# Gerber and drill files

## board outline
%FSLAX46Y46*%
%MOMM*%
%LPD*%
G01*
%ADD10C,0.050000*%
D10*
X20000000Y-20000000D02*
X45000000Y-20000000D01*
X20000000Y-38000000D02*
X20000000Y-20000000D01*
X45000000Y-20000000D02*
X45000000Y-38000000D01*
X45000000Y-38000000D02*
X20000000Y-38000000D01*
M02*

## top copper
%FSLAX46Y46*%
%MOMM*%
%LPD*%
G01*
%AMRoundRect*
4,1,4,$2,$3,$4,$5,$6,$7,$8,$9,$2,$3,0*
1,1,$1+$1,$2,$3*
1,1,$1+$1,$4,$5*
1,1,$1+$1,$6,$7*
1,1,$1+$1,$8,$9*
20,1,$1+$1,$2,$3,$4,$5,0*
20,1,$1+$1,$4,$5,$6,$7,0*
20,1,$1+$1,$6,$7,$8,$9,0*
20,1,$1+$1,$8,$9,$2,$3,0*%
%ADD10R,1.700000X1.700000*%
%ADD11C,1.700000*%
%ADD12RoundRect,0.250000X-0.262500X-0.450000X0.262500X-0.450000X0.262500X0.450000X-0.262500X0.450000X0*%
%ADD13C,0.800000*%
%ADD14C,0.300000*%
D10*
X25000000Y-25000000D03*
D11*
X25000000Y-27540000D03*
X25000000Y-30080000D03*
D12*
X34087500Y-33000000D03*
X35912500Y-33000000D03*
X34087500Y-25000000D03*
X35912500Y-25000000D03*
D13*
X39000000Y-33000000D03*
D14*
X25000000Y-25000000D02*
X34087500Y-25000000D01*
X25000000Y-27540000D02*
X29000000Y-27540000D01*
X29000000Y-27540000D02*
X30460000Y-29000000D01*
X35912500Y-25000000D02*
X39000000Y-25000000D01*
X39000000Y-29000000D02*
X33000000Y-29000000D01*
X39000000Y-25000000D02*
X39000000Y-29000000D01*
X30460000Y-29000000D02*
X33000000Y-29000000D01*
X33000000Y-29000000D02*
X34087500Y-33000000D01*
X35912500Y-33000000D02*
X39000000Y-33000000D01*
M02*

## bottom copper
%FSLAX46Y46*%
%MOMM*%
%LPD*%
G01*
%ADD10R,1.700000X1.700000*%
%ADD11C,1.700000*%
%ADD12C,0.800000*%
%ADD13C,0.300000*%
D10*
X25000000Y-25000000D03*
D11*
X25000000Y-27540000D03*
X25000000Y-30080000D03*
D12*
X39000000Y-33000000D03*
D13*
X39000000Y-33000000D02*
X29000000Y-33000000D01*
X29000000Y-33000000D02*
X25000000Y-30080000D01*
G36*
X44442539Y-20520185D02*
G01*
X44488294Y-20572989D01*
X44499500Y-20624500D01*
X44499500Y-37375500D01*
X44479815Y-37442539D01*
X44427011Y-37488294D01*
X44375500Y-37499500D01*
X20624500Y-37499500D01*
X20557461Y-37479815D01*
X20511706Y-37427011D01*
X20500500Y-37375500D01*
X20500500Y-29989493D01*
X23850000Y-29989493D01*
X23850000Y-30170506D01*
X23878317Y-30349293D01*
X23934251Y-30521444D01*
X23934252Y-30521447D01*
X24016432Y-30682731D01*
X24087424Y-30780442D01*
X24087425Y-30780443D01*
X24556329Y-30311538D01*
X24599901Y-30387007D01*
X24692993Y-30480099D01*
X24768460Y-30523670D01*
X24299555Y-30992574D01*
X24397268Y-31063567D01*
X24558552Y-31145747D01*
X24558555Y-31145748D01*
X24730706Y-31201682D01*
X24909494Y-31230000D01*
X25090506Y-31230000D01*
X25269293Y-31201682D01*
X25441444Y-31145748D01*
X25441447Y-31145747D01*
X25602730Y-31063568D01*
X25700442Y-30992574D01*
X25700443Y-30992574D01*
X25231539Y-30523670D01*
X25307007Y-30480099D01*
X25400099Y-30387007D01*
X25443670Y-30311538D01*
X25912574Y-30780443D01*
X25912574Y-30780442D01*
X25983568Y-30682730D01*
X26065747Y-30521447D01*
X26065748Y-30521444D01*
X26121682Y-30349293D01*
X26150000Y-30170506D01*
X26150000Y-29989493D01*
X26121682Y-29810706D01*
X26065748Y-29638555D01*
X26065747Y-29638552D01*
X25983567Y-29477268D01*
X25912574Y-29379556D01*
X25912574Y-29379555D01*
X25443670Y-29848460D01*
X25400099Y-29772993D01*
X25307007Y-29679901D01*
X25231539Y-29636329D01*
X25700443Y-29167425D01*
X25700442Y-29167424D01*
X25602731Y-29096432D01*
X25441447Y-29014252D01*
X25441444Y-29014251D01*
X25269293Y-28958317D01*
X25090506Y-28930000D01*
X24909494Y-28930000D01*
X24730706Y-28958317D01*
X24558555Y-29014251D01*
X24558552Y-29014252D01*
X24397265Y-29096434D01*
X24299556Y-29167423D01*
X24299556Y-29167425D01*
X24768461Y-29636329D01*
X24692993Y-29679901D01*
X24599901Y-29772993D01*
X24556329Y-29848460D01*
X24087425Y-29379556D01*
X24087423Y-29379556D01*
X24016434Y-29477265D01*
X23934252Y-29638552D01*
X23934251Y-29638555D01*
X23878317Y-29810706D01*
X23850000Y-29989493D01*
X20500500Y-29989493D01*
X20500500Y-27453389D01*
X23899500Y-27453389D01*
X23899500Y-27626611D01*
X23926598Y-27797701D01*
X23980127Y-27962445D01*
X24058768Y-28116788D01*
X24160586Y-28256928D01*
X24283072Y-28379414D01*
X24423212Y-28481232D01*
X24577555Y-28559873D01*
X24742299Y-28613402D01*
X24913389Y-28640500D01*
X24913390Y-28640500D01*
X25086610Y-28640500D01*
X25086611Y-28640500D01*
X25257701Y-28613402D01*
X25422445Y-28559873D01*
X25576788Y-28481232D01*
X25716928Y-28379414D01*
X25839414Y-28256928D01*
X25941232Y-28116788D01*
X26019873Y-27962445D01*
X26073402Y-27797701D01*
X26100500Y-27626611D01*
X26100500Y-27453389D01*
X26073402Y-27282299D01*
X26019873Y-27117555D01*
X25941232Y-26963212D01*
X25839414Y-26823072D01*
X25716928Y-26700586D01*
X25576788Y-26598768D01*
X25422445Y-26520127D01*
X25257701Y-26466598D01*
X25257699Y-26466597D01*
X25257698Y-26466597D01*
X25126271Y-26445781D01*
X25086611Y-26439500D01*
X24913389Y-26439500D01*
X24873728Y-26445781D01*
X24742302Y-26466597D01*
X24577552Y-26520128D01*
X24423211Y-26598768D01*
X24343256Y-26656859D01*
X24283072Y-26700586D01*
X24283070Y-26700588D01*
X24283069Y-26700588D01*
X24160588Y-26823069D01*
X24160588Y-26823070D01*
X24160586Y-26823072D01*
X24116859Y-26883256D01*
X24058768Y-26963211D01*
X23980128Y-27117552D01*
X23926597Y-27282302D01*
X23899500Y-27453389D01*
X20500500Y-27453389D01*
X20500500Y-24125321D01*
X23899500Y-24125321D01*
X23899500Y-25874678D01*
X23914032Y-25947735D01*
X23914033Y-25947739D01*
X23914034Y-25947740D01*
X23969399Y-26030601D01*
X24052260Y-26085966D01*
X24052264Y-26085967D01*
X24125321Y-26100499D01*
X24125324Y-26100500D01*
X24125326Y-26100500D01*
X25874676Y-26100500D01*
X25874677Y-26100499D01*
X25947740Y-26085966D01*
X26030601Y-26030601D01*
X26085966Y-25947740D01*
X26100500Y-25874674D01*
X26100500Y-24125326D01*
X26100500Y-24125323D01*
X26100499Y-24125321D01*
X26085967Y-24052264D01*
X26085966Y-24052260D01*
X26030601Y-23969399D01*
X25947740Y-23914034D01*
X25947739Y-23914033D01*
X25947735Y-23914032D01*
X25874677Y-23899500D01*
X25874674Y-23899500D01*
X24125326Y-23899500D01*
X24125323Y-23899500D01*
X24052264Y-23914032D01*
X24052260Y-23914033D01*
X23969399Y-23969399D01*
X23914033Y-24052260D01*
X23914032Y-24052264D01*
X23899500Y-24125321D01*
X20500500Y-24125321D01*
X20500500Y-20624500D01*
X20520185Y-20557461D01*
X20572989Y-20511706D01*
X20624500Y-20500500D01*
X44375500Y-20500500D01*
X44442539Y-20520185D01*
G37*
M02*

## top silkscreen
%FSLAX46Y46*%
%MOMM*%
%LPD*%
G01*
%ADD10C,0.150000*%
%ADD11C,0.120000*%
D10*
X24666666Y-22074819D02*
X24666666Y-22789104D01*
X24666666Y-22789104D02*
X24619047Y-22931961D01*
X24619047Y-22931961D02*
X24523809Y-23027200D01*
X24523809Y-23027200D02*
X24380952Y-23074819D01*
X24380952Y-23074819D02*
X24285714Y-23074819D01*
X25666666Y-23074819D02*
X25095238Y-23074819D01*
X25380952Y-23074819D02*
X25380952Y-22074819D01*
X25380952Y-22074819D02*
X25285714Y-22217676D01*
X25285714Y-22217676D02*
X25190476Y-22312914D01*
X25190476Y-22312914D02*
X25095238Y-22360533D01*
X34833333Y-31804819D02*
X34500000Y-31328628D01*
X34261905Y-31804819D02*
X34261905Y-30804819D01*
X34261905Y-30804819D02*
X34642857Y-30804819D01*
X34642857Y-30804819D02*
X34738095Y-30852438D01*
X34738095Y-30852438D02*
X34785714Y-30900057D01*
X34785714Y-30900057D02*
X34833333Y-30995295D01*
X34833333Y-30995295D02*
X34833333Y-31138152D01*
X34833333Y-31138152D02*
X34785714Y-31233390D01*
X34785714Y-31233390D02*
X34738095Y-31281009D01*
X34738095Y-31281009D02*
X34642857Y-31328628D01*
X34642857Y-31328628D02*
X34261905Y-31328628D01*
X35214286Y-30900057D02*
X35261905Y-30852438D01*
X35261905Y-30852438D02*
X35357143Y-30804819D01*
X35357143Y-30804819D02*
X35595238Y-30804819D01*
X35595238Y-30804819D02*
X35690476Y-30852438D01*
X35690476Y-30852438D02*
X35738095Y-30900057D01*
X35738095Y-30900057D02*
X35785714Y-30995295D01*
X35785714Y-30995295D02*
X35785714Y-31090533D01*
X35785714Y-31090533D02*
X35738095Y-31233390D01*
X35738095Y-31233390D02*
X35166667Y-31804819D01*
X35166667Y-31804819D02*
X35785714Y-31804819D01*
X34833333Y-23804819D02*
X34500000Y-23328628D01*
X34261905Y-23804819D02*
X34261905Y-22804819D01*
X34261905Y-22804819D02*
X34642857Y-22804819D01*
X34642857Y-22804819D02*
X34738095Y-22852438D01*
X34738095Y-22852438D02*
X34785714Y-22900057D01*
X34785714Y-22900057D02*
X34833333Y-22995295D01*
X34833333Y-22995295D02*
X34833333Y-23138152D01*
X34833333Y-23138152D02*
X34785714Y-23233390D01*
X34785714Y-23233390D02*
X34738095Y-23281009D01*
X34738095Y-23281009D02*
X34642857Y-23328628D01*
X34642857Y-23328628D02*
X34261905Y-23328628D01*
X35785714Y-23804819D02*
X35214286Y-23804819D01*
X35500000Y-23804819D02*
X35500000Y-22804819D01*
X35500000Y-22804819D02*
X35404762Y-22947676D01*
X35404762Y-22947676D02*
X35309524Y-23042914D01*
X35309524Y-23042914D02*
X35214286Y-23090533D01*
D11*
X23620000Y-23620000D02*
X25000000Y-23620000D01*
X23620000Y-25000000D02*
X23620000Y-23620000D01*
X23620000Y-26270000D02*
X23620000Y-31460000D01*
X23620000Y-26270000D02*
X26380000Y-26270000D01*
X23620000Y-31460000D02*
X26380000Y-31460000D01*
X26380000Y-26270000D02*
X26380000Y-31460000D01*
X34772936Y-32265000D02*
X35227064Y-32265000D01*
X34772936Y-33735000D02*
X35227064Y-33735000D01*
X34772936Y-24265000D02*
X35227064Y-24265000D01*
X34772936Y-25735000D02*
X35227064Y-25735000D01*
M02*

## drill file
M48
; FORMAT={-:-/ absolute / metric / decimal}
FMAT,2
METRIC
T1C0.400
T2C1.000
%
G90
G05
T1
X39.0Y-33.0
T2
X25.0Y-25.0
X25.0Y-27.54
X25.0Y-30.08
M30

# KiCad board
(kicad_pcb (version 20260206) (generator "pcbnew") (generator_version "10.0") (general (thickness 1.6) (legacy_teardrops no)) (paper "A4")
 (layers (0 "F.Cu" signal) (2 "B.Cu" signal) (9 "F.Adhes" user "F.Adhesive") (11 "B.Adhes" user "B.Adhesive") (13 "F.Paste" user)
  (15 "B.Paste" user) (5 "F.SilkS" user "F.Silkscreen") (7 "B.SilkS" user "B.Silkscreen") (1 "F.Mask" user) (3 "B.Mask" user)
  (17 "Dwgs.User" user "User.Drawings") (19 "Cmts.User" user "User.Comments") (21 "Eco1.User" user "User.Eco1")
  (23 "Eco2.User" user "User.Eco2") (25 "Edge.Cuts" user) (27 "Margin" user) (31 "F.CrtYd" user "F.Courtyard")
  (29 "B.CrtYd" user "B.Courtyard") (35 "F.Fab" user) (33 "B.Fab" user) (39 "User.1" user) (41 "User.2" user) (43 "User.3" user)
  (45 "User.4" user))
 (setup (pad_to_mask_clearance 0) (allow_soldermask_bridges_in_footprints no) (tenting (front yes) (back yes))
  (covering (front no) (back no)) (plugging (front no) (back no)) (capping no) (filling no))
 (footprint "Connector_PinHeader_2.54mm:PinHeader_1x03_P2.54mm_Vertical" (layer "F.Cu") (at 25 25)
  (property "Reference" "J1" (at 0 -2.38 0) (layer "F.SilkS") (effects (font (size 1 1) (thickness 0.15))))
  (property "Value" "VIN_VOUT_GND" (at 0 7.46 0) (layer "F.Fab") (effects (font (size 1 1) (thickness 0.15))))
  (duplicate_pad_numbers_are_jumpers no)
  (fp_line (start -1.38 -1.38) (end 0 -1.38) (stroke (width 0.12) (type solid)) (layer "F.SilkS"))
  (fp_line (start -1.38 0) (end -1.38 -1.38) (stroke (width 0.12) (type solid)) (layer "F.SilkS"))
  (fp_line (start -1.38 1.27) (end -1.38 6.46) (stroke (width 0.12) (type solid)) (layer "F.SilkS"))
  (fp_line (start -1.38 1.27) (end 1.38 1.27) (stroke (width 0.12) (type solid)) (layer "F.SilkS"))
  (fp_line (start -1.38 6.46) (end 1.38 6.46) (stroke (width 0.12) (type solid)) (layer "F.SilkS"))
  (fp_line (start 1.38 1.27) (end 1.38 6.46) (stroke (width 0.12) (type solid)) (layer "F.SilkS"))
  (pad "1" thru_hole rect (at 0 0) (size 1.7 1.7) (drill 1) (layers "*.Cu" "*.Mask") (remove_unused_layers no) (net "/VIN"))
  (pad "2" thru_hole circle (at 0 2.54) (size 1.7 1.7) (drill 1) (layers "*.Cu" "*.Mask") (remove_unused_layers no) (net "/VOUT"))
  (pad "3" thru_hole circle (at 0 5.08) (size 1.7 1.7) (drill 1) (layers "*.Cu" "*.Mask") (remove_unused_layers no) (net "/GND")))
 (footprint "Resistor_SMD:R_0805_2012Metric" (layer "F.Cu") (at 35 33)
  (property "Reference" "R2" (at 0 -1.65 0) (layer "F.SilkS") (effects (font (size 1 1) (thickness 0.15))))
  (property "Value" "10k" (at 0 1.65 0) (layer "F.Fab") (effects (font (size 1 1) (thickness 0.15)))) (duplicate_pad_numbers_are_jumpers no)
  (fp_line (start -0.227064 -0.735) (end 0.227064 -0.735) (stroke (width 0.12) (type solid)) (layer "F.SilkS"))
  (fp_line (start -0.227064 0.735) (end 0.227064 0.735) (stroke (width 0.12) (type solid)) (layer "F.SilkS"))
  (pad "1" smd roundrect (at -0.9125 0) (size 1.025 1.4) (layers "F.Cu" "F.Mask" "F.Paste") (roundrect_rratio 0.243902) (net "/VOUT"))
  (pad "2" smd roundrect (at 0.9125 0) (size 1.025 1.4) (layers "F.Cu" "F.Mask" "F.Paste") (roundrect_rratio 0.243902) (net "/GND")))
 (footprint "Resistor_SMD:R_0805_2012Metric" (layer "F.Cu") (at 35 25)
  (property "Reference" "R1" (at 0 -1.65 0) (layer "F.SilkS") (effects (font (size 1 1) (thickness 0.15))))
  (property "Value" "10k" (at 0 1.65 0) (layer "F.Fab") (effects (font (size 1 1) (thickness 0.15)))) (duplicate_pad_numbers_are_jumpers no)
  (fp_line (start -0.227064 -0.735) (end 0.227064 -0.735) (stroke (width 0.12) (type solid)) (layer "F.SilkS"))
  (fp_line (start -0.227064 0.735) (end 0.227064 0.735) (stroke (width 0.12) (type solid)) (layer "F.SilkS"))
  (pad "1" smd roundrect (at -0.9125 0) (size 1.025 1.4) (layers "F.Cu" "F.Mask" "F.Paste") (roundrect_rratio 0.243902) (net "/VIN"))
  (pad "2" smd roundrect (at 0.9125 0) (size 1.025 1.4) (layers "F.Cu" "F.Mask" "F.Paste") (roundrect_rratio 0.243902) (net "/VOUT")))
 (gr_line (start 20 20) (end 45 20) (stroke (width 0.05) (type default)) (layer "Edge.Cuts"))
 (gr_line (start 20 38) (end 20 20) (stroke (width 0.05) (type default)) (layer "Edge.Cuts"))
 (gr_line (start 45 20) (end 45 38) (stroke (width 0.05) (type default)) (layer "Edge.Cuts"))
 (gr_line (start 45 38) (end 20 38) (stroke (width 0.05) (type default)) (layer "Edge.Cuts"))
 (segment (start 25 25) (end 34.0875 25) (width 0.3) (layer "F.Cu") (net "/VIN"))
 (segment (start 25 27.54) (end 29 27.54) (width 0.3) (layer "F.Cu") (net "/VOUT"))
 (segment (start 29 27.54) (end 30.46 29) (width 0.3) (layer "F.Cu") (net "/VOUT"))
 (segment (start 35.9125 25) (end 39 25) (width 0.3) (layer "F.Cu") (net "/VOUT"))
 (segment (start 39 29) (end 33 29) (width 0.3) (layer "F.Cu") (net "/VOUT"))
 (segment (start 39 25) (end 39 29) (width 0.3) (layer "F.Cu") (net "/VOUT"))
 (segment (start 30.46 29) (end 33 29) (width 0.3) (layer "F.Cu") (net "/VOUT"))
 (segment (start 33 29) (end 34.0875 33) (width 0.3) (layer "F.Cu") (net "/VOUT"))
 (segment (start 35.9125 33) (end 39 33) (width 0.3) (layer "F.Cu") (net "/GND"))
 (via (at 39 33) (size 0.8) (drill 0.4) (layers "F.Cu" "B.Cu") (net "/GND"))
 (segment (start 39 33) (end 29 33) (width 0.3) (layer "B.Cu") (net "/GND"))
 (segment (start 29 33) (end 25 30.08) (width 0.3) (layer "B.Cu") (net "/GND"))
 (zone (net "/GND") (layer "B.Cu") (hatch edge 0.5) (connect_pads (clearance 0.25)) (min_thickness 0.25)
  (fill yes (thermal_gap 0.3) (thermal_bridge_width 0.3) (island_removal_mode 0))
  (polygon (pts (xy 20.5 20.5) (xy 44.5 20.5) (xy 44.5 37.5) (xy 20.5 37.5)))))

